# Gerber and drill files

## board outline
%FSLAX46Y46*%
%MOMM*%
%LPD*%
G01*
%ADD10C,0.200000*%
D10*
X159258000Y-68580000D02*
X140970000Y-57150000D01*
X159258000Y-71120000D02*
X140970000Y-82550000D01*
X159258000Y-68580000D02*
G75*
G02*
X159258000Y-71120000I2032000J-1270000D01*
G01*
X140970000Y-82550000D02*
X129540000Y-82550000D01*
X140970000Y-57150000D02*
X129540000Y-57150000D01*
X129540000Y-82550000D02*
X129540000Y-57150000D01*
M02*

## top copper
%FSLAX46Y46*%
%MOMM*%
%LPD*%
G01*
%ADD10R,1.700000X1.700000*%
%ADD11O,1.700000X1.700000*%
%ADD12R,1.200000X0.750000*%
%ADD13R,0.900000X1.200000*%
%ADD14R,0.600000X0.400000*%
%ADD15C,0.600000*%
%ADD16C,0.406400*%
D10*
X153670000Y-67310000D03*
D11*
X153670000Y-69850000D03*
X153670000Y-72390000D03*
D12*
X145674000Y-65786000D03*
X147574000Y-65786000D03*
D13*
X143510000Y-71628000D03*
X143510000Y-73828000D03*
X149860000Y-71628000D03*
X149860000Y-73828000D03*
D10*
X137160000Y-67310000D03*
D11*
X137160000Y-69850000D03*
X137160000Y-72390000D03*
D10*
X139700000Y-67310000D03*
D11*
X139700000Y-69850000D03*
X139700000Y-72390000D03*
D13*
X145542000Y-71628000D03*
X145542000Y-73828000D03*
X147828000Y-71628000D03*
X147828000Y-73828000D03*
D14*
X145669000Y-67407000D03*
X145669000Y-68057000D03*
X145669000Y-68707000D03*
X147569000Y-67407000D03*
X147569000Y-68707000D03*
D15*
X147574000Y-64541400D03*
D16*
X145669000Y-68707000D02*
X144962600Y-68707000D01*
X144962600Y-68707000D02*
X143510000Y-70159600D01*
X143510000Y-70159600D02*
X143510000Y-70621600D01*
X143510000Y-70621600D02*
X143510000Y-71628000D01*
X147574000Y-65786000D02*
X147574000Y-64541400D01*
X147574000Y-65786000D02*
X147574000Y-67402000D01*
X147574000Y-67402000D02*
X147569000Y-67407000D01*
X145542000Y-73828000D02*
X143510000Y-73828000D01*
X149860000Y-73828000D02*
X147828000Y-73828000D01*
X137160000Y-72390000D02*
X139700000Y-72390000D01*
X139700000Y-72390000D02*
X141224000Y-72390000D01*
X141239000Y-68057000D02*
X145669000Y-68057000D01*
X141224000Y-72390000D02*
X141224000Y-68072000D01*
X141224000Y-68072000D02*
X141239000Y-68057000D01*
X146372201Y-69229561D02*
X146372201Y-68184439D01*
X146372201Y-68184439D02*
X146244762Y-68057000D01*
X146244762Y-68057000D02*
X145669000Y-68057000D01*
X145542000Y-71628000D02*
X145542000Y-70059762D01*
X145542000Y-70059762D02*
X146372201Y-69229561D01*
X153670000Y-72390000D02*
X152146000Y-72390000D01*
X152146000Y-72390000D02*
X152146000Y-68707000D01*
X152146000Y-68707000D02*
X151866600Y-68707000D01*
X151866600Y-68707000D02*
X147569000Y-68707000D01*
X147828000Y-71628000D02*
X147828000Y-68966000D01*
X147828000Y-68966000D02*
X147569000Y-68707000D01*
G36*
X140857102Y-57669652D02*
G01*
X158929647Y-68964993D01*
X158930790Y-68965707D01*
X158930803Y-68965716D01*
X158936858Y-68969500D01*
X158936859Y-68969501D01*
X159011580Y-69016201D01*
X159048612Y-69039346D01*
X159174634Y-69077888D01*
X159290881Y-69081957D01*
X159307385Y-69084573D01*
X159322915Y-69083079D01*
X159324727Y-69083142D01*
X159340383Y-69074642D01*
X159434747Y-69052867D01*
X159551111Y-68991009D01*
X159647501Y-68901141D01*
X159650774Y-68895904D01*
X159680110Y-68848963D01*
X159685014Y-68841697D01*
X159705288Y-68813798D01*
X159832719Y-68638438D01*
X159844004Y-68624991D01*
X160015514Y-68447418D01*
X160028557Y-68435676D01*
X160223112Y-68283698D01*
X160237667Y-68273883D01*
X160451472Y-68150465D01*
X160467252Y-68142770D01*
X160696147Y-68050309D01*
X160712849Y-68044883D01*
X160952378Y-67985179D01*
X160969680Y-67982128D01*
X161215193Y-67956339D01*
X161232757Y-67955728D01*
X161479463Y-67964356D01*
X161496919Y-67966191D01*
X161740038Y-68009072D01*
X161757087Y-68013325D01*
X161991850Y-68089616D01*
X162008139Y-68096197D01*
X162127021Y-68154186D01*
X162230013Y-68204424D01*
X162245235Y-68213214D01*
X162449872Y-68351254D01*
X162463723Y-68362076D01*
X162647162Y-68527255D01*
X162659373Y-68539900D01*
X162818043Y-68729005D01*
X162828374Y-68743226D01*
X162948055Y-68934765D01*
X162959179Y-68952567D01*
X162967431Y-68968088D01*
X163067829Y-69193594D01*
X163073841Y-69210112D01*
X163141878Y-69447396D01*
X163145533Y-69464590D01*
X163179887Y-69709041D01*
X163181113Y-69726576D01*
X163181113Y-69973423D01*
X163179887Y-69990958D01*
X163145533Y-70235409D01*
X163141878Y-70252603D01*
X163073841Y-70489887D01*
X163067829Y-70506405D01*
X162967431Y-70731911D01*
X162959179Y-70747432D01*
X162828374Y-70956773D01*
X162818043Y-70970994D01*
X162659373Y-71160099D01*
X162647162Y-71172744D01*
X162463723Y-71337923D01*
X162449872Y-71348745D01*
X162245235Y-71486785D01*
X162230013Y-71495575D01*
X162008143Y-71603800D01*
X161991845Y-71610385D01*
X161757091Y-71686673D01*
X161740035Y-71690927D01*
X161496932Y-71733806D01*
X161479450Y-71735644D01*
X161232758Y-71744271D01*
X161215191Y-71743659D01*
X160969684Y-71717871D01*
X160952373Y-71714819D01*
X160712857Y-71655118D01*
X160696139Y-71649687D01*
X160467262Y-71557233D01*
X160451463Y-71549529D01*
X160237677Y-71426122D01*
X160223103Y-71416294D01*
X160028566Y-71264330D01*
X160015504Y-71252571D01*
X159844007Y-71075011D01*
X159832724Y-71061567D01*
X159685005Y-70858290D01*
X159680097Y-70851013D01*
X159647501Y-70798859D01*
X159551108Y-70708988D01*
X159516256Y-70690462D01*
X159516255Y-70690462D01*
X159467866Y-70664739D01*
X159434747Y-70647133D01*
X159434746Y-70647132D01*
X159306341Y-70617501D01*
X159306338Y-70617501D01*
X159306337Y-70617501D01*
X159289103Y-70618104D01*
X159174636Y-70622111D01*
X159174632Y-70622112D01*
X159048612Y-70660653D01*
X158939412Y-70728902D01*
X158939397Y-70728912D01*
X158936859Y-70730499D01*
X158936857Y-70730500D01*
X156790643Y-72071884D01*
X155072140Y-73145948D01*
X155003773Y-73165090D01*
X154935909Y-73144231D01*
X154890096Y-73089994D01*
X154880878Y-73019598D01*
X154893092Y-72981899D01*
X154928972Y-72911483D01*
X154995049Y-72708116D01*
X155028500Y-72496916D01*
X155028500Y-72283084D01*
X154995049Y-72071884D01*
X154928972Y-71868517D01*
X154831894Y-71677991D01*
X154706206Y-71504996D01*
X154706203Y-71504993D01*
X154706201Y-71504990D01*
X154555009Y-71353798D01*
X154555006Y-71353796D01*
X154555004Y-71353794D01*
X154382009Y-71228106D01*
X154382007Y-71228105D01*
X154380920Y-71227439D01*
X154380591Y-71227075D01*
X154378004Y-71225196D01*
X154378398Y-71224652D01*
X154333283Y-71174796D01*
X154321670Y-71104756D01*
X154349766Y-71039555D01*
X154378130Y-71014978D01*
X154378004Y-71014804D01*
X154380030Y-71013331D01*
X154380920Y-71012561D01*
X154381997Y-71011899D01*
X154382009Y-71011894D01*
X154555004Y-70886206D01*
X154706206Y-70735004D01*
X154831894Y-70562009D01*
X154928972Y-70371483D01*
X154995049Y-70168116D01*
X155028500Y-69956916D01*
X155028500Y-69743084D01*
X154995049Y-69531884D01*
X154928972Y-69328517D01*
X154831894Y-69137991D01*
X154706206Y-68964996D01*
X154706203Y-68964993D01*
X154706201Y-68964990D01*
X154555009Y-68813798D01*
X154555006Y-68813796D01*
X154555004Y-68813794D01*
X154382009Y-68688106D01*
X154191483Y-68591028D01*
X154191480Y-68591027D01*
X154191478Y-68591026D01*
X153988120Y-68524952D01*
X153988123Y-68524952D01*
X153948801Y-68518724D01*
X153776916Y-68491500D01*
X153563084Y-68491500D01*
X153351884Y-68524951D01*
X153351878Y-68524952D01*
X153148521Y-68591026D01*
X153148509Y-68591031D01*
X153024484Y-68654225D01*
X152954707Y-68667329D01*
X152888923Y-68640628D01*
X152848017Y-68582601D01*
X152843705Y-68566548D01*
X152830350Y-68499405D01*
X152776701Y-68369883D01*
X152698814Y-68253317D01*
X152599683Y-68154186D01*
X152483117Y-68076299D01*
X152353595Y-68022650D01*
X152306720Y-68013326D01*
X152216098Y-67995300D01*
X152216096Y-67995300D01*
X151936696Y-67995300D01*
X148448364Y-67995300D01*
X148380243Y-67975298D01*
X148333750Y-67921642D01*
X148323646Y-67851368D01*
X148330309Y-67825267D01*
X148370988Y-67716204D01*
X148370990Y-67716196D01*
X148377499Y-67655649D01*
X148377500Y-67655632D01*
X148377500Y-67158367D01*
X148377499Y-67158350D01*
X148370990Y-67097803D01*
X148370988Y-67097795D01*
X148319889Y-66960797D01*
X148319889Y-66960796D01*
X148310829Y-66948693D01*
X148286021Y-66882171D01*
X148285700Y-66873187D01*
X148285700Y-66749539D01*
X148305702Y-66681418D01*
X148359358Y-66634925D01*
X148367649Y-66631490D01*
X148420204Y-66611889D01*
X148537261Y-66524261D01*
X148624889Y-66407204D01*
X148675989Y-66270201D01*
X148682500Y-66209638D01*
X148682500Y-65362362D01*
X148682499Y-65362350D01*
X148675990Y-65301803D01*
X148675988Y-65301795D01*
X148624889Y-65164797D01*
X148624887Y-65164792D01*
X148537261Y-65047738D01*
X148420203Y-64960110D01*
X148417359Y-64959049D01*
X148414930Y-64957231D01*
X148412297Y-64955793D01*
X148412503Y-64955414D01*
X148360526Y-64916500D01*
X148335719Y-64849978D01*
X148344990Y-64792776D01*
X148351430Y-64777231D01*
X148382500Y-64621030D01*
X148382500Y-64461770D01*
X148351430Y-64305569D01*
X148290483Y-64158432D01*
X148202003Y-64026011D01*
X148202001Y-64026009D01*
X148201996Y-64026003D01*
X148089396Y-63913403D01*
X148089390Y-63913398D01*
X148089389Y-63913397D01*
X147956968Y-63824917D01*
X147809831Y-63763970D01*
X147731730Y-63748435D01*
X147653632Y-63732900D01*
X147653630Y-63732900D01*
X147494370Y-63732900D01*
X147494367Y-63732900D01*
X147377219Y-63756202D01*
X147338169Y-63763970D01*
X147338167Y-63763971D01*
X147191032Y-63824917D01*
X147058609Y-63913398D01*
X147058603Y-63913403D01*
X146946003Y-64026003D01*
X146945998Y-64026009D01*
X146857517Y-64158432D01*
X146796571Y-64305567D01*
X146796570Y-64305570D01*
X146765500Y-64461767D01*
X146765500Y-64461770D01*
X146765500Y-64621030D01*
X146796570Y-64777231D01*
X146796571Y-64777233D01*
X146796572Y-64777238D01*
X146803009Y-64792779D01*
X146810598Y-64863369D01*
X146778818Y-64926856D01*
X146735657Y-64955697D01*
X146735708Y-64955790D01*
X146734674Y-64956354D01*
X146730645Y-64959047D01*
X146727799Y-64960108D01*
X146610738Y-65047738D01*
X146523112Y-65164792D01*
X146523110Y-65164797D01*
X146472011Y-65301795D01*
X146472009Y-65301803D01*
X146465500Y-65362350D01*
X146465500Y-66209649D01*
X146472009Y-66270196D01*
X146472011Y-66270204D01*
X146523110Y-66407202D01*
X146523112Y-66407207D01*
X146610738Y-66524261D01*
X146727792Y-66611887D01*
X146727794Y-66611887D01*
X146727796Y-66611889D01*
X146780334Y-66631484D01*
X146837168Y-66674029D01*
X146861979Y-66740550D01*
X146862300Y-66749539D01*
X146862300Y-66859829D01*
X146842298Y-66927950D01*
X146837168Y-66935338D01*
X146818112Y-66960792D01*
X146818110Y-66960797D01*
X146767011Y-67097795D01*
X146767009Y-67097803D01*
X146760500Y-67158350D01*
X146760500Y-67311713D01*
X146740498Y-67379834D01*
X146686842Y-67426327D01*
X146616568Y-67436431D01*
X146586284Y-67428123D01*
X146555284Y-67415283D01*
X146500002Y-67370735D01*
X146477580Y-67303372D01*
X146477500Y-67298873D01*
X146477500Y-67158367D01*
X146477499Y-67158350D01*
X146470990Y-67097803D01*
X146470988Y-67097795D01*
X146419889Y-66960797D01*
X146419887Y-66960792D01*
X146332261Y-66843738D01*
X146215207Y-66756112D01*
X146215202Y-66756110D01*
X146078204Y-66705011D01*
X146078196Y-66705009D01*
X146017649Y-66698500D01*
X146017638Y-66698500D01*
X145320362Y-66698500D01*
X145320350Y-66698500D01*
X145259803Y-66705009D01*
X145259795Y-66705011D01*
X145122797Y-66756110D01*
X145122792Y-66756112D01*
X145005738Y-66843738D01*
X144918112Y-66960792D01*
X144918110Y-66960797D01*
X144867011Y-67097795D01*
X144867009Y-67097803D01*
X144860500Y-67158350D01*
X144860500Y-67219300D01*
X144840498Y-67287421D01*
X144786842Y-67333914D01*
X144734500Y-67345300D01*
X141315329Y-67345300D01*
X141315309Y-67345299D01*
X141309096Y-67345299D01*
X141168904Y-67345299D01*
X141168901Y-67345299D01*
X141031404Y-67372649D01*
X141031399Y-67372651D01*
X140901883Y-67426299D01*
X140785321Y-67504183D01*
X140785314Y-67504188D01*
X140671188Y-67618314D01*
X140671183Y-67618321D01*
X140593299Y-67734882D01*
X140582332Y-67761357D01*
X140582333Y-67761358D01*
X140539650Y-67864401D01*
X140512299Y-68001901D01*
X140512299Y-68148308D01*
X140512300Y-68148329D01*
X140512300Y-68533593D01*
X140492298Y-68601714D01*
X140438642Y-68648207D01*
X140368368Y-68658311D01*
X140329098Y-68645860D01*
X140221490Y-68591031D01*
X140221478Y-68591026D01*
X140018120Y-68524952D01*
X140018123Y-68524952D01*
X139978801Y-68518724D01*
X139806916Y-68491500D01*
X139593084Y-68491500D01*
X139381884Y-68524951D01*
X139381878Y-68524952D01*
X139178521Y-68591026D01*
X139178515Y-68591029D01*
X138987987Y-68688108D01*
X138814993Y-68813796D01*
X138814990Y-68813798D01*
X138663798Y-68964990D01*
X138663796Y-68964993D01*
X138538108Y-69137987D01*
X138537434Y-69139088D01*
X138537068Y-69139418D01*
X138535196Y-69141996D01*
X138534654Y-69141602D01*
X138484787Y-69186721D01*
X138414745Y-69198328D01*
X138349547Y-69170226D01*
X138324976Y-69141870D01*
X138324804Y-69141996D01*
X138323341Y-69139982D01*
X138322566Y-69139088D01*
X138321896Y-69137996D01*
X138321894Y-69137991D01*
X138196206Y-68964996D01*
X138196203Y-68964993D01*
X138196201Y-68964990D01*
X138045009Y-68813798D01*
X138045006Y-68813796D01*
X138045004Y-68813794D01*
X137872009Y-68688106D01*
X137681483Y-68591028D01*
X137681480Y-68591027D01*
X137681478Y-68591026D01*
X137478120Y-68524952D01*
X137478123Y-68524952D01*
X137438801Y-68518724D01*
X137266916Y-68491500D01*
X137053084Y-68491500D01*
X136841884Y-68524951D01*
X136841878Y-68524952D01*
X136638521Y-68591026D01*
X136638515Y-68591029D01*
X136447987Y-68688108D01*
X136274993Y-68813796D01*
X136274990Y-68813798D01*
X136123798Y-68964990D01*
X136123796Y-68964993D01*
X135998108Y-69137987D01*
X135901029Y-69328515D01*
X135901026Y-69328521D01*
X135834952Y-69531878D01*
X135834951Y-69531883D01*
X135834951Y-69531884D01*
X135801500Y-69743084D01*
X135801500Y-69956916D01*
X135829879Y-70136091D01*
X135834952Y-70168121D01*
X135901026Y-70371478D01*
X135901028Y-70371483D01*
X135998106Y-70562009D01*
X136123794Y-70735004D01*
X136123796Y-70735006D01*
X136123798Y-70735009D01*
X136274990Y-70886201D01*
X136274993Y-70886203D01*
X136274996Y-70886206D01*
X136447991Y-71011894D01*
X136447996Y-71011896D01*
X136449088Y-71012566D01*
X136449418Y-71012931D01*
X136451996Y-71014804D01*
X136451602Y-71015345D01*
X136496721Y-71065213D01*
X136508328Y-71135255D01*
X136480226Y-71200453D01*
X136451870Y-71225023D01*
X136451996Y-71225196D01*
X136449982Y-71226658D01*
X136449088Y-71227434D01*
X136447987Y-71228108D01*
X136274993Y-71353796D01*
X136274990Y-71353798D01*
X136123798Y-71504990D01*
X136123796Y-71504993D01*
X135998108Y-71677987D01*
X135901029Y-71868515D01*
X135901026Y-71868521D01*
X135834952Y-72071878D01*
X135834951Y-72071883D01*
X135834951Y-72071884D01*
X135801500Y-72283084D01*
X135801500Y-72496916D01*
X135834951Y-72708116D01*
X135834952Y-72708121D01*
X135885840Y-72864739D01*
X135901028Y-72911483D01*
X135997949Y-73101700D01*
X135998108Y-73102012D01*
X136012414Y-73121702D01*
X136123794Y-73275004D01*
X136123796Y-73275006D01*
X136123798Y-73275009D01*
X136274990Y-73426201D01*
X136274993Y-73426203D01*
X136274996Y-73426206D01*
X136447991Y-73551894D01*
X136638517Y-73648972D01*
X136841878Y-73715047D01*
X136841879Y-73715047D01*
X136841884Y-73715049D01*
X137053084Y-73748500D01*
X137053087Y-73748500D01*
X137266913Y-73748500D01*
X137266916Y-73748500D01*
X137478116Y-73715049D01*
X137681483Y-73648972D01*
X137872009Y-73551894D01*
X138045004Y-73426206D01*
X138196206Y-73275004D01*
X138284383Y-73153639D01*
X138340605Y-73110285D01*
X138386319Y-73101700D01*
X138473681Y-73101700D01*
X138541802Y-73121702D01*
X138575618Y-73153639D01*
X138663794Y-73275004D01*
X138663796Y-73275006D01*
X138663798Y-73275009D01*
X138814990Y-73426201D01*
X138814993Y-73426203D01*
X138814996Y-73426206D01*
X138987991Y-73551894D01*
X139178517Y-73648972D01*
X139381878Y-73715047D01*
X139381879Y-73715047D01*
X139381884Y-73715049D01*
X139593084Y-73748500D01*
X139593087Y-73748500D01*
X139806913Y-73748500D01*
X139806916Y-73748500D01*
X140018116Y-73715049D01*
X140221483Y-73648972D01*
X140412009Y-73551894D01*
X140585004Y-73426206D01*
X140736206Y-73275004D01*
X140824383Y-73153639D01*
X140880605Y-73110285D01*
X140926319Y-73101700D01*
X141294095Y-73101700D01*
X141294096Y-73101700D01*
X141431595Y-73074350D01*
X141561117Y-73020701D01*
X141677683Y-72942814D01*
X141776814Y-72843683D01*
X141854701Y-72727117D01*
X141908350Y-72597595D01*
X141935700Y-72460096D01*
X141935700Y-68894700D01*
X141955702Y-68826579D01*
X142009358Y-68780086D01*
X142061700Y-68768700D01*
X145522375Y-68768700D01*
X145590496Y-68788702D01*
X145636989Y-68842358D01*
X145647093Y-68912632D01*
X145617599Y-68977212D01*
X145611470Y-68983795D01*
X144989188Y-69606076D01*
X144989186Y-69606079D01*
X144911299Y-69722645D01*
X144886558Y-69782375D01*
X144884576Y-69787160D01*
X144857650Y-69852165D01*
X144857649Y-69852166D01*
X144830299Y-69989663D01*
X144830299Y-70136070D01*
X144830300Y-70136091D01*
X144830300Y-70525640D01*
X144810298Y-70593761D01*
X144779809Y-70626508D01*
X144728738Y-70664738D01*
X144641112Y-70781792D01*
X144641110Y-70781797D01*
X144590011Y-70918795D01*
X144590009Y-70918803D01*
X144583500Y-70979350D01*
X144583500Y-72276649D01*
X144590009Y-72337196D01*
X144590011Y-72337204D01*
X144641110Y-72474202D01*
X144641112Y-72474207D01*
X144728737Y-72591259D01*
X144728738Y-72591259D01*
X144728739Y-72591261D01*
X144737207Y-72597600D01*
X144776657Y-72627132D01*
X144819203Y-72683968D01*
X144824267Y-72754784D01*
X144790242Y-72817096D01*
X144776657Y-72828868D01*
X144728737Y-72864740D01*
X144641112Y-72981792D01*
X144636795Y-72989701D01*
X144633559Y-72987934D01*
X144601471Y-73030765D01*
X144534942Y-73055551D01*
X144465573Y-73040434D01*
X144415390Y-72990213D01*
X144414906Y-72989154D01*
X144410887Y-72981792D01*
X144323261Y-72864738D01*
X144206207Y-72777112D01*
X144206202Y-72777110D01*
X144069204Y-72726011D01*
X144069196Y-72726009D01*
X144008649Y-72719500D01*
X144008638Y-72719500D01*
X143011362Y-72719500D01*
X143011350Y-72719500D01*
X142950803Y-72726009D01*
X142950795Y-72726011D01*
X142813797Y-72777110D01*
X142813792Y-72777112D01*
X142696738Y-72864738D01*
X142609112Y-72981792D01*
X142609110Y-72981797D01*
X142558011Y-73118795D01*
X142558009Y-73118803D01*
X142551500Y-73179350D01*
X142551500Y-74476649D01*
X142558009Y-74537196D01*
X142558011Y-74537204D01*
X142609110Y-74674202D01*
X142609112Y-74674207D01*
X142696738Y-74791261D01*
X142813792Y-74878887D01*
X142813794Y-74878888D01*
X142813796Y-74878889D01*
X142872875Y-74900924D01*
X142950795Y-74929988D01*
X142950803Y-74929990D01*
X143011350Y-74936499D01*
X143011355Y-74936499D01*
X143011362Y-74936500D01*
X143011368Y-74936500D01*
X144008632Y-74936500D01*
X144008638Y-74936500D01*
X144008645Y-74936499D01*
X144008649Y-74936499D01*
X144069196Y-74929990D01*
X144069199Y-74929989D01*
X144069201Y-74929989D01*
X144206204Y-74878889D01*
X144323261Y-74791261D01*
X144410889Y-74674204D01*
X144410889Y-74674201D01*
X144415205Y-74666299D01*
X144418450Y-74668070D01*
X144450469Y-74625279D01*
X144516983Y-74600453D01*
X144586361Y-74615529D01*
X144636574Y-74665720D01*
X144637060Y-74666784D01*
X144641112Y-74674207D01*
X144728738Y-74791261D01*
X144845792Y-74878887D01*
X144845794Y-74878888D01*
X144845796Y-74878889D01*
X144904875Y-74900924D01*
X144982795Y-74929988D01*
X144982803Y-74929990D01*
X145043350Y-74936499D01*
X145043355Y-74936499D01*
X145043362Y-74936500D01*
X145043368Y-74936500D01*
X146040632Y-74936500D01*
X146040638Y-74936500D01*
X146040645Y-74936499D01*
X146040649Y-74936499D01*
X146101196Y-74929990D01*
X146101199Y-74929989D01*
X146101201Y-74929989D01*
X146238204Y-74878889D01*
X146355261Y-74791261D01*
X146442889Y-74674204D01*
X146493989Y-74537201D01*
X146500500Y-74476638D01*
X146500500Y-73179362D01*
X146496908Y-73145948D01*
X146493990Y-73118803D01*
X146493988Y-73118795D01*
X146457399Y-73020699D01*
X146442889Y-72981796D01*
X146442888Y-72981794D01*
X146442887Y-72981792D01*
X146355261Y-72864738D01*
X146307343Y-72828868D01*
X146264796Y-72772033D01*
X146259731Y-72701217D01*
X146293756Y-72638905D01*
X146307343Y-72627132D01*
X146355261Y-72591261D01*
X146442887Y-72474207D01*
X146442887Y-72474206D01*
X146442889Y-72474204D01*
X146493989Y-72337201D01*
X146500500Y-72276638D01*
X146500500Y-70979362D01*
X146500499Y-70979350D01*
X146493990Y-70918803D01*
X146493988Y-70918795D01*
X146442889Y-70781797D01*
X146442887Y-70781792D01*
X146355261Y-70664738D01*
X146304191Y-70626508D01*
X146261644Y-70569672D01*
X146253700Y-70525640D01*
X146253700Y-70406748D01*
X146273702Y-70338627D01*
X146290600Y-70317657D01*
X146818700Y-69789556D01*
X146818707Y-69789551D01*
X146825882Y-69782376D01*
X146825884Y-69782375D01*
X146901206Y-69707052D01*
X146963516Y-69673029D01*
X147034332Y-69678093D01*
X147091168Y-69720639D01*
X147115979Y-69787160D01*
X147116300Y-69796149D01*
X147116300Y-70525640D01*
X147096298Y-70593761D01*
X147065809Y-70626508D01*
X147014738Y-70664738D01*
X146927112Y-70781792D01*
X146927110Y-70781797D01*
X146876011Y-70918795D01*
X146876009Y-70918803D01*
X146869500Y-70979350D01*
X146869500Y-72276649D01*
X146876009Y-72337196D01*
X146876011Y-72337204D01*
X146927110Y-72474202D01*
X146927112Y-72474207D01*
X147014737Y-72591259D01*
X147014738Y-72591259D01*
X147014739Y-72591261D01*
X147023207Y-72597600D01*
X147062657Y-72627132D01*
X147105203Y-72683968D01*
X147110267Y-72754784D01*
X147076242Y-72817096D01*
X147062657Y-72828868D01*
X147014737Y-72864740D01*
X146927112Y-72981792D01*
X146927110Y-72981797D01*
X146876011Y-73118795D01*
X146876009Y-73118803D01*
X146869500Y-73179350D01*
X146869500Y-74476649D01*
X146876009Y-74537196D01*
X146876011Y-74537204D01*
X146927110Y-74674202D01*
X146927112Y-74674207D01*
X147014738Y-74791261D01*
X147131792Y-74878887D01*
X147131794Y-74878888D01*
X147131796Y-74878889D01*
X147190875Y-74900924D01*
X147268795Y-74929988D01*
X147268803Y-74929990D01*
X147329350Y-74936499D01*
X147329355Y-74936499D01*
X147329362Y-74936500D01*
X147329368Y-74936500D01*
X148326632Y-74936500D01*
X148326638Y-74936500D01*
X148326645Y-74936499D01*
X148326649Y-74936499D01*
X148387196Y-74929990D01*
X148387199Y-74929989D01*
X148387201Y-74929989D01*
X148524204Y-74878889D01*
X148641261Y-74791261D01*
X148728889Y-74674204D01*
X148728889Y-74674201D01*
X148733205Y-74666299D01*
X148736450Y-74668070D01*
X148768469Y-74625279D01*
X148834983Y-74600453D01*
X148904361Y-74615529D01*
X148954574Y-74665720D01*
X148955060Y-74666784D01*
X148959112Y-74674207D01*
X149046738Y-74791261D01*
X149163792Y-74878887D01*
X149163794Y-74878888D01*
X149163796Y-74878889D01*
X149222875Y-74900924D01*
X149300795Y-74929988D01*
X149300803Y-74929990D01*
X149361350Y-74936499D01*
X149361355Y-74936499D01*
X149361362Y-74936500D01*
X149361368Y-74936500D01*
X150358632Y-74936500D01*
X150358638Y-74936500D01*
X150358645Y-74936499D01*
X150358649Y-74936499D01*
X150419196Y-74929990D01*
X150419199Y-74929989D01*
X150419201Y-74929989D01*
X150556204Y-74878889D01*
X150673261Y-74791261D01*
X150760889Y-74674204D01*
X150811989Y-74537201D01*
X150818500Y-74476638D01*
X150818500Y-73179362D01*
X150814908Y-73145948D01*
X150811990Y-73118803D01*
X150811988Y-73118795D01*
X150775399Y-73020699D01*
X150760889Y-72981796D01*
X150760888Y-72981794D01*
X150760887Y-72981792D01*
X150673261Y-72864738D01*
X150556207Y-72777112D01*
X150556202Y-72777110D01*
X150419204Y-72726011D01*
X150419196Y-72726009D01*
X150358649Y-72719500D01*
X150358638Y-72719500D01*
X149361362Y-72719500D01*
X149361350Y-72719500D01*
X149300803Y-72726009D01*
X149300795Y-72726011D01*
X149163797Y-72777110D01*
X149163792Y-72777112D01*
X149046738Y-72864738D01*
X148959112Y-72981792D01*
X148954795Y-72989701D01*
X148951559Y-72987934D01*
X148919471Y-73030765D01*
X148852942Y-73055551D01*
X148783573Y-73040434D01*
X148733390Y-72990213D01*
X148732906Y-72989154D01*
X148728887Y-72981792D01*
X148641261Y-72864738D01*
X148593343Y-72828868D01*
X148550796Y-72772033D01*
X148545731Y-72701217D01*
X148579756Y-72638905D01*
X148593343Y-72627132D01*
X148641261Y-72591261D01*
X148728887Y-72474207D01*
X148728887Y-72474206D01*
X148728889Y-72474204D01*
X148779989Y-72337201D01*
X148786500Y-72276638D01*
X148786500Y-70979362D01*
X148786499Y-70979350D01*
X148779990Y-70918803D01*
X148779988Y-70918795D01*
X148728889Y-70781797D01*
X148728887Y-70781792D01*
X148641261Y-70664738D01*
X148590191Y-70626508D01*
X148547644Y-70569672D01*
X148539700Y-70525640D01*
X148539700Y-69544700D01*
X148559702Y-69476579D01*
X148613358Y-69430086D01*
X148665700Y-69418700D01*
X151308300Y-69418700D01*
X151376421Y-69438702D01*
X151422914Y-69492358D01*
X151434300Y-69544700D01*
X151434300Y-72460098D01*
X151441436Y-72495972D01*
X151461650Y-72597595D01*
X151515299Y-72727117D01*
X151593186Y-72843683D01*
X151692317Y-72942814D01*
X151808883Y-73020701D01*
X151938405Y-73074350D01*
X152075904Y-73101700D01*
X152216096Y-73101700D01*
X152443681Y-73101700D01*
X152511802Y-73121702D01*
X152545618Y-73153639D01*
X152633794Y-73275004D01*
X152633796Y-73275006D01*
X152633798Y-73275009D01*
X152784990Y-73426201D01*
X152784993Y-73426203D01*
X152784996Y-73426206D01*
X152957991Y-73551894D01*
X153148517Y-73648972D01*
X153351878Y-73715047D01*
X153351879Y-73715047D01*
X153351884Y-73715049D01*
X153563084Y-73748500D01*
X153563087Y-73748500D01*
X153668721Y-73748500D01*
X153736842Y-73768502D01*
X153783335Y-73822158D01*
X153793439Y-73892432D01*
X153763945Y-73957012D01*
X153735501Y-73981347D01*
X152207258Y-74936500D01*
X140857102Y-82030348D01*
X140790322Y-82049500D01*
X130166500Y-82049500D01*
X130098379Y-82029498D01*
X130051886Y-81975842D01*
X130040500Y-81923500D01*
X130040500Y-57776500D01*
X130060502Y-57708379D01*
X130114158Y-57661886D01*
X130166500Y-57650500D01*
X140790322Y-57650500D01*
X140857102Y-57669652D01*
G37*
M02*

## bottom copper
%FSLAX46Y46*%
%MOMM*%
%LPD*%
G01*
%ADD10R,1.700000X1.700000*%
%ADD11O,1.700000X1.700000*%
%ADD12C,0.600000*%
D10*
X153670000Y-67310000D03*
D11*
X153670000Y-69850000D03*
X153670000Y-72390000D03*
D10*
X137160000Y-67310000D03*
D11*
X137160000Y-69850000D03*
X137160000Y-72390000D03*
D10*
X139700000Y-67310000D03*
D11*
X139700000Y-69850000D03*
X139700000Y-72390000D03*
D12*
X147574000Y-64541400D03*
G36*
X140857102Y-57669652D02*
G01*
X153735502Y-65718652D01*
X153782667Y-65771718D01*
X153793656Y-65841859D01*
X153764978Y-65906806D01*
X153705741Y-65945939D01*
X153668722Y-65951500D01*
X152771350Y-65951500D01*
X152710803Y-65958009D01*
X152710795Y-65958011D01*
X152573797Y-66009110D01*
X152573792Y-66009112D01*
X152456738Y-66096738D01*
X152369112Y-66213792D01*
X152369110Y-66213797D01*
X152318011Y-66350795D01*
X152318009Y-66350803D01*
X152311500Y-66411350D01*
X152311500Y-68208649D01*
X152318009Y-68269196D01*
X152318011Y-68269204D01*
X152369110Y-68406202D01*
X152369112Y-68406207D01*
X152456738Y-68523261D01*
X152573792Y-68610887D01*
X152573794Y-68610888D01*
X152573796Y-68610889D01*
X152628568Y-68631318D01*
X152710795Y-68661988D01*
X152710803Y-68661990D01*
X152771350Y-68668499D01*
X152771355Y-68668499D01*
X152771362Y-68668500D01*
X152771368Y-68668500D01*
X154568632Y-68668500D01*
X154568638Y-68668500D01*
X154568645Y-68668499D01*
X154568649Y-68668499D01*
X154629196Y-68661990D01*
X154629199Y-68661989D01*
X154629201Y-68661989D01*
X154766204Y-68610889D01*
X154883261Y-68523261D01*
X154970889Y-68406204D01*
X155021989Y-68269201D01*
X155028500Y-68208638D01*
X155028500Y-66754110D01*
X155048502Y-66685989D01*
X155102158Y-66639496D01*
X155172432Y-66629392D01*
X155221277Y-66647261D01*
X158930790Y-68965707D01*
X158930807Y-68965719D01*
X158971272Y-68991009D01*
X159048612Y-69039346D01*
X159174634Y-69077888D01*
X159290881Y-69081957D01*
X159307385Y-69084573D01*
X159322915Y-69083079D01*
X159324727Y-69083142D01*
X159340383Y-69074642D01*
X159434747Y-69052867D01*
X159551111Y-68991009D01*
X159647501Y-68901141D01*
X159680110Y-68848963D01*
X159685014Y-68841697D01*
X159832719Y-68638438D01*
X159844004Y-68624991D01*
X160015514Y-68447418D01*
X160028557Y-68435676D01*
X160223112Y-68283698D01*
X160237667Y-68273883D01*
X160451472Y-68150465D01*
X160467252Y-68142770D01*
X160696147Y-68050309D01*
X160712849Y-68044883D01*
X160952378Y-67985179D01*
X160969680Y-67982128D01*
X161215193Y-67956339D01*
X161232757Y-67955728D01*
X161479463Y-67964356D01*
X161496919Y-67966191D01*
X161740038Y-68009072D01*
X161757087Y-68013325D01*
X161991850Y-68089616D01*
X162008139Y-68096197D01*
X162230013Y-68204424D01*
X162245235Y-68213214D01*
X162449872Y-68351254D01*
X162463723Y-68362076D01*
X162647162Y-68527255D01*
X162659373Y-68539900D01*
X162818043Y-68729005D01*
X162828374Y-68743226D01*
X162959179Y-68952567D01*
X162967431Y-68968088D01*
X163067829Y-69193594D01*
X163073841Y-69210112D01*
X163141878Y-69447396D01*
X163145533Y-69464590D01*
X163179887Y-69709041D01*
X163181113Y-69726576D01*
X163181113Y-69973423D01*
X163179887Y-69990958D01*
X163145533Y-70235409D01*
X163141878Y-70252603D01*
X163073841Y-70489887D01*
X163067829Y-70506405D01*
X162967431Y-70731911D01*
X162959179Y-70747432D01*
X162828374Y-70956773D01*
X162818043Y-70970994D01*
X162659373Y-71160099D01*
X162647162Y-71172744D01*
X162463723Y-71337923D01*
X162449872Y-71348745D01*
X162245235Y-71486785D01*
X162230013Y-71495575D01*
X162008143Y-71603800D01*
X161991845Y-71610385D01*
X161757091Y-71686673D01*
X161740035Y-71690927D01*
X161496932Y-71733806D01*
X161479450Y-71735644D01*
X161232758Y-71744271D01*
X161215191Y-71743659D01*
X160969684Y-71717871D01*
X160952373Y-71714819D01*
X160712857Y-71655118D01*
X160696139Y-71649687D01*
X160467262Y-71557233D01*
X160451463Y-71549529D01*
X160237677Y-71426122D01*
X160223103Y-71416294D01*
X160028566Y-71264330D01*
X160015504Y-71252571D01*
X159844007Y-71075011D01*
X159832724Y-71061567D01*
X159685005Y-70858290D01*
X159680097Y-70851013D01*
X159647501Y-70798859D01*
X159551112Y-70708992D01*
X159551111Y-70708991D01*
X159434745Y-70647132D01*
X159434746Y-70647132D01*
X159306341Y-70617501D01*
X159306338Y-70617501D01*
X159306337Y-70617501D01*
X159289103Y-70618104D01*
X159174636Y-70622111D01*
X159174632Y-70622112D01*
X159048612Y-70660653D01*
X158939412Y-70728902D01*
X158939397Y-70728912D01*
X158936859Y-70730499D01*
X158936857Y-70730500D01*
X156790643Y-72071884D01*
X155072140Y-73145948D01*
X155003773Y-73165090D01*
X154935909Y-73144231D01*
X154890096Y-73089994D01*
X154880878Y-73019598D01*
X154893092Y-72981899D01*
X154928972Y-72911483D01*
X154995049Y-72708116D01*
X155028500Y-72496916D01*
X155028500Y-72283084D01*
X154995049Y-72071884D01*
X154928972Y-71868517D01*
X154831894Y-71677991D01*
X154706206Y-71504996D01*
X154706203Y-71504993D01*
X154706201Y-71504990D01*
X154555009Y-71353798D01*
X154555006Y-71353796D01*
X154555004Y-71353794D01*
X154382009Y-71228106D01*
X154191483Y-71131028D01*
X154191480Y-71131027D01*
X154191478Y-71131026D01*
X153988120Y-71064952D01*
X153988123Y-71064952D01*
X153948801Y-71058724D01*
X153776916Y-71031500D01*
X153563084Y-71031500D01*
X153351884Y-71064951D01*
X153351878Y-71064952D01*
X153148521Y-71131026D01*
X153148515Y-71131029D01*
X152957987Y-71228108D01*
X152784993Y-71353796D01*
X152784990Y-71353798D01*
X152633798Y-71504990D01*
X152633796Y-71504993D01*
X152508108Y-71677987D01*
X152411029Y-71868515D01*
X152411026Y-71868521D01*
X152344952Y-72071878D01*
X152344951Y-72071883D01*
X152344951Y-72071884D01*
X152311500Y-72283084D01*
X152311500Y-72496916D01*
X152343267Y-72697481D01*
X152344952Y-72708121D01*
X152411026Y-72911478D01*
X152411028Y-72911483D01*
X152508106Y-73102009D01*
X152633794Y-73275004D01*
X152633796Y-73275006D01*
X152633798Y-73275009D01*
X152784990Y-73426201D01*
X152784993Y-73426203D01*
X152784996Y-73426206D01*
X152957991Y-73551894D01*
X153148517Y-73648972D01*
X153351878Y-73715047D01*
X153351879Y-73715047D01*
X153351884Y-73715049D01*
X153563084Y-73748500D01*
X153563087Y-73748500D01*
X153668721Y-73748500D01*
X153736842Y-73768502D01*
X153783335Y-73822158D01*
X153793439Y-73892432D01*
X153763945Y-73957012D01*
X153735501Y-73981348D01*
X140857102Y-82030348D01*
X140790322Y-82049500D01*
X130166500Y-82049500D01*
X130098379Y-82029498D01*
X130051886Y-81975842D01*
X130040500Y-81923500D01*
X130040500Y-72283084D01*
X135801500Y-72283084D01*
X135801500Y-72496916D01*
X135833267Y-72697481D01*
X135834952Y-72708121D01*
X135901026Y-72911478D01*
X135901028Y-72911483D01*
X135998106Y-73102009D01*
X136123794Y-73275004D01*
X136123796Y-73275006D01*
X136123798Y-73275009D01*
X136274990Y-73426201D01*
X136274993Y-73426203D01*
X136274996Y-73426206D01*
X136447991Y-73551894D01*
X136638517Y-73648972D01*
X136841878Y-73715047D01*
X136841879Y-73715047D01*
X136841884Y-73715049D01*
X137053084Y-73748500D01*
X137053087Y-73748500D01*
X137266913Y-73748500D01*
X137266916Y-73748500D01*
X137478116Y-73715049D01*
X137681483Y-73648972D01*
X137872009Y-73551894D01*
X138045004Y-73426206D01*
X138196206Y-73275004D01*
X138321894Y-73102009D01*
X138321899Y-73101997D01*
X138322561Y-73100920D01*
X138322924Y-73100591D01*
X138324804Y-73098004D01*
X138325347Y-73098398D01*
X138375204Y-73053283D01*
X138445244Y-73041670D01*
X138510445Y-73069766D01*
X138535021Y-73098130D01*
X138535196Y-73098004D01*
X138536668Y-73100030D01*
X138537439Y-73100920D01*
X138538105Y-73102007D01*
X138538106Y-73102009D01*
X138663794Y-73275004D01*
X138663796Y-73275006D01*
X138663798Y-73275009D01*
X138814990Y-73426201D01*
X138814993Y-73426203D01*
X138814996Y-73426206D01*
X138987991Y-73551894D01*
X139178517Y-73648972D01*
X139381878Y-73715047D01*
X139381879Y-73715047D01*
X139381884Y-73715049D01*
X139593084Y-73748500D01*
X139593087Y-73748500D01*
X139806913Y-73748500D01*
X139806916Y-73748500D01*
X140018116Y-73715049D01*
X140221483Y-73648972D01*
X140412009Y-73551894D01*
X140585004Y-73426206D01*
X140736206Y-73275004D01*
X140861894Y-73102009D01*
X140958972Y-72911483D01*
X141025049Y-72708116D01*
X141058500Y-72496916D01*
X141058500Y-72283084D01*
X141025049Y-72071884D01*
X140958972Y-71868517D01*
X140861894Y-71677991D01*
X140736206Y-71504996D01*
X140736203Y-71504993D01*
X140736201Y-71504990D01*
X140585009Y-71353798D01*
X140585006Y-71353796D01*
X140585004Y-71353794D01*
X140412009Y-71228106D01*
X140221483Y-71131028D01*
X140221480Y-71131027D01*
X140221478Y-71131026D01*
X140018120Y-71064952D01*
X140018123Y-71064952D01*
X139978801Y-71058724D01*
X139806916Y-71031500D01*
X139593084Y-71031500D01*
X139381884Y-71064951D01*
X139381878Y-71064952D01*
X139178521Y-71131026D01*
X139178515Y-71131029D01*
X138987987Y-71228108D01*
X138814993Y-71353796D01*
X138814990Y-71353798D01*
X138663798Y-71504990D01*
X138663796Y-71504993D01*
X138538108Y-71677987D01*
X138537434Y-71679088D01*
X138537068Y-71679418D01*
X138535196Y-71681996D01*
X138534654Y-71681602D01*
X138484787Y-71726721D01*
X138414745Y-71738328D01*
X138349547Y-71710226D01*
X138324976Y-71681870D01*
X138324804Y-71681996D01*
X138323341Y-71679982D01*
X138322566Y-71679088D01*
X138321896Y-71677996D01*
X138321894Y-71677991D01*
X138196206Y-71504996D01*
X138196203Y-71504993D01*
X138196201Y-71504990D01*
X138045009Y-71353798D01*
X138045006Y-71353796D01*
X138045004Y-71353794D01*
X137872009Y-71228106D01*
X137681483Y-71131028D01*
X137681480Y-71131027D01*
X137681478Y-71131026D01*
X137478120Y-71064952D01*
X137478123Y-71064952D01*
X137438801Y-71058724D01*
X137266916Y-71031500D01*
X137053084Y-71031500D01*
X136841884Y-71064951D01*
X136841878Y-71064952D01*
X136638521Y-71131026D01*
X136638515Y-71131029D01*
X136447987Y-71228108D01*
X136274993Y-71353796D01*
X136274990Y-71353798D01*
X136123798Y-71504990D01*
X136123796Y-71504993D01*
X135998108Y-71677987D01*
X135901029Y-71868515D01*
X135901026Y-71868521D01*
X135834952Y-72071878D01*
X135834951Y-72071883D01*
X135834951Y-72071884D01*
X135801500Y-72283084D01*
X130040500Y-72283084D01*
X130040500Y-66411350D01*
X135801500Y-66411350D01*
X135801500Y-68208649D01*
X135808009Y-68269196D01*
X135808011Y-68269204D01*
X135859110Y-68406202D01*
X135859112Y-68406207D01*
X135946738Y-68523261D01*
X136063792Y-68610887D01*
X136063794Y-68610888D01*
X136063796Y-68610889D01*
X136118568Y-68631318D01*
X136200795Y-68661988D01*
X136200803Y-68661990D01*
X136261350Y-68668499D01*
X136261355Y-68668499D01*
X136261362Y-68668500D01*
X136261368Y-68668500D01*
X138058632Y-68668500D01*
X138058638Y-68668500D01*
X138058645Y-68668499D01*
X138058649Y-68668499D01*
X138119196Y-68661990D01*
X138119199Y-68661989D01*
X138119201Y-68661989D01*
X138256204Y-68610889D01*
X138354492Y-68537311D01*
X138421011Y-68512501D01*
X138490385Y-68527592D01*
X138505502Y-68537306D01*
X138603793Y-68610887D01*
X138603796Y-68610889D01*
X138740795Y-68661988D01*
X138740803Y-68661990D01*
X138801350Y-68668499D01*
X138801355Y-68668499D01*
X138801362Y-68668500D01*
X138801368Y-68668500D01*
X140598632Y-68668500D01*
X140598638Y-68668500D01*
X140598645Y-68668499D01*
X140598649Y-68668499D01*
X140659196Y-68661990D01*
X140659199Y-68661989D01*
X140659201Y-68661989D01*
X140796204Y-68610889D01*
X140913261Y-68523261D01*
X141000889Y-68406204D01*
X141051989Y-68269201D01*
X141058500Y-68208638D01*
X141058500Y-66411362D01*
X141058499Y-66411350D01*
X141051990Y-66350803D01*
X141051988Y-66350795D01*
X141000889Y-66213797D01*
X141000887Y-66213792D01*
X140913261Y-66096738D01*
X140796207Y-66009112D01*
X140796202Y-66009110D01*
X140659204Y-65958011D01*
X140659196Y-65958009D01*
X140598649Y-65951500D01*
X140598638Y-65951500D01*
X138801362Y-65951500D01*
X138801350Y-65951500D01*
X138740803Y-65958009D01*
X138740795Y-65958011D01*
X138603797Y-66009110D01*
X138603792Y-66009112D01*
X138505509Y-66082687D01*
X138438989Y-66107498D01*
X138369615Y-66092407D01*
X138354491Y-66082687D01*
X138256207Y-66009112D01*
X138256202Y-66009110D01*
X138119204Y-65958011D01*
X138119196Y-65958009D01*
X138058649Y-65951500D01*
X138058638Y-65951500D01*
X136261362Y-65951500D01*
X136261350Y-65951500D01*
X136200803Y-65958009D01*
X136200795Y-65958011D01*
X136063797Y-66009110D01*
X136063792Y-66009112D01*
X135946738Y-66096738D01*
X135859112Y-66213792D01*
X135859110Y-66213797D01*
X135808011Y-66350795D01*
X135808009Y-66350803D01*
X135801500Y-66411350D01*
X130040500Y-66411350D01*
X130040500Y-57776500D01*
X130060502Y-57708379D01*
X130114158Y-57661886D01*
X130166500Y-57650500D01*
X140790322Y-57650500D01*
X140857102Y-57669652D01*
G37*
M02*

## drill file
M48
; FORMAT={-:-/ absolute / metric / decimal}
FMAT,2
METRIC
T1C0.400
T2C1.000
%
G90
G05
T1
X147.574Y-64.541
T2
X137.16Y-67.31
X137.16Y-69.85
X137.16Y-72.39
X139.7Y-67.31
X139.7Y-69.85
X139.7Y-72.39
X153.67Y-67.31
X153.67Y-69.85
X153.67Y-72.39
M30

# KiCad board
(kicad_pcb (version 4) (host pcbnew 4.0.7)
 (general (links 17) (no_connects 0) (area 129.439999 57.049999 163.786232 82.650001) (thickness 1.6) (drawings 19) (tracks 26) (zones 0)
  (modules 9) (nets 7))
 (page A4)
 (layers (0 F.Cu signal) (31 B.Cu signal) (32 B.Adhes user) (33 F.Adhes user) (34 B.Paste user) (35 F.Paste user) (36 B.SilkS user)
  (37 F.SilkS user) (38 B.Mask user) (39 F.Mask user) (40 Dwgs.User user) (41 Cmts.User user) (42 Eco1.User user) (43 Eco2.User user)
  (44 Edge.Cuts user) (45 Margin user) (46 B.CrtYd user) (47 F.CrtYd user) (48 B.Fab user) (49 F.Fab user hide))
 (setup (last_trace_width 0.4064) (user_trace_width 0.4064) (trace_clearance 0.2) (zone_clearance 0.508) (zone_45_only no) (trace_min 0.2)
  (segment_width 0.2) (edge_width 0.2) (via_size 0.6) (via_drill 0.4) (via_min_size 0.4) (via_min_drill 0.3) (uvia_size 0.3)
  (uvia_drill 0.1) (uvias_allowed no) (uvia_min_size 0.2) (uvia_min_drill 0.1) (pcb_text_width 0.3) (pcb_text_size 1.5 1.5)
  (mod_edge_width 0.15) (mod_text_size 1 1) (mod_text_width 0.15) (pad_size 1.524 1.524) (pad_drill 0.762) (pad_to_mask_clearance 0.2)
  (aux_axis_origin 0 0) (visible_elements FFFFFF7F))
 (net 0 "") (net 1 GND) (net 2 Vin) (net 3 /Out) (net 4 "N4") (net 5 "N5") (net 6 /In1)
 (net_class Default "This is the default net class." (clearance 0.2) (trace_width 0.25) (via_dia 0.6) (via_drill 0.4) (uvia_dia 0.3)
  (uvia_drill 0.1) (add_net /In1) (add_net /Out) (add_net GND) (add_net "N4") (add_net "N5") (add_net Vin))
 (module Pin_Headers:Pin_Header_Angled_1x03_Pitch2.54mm (layer F.Cu) (at 153.67 67.31)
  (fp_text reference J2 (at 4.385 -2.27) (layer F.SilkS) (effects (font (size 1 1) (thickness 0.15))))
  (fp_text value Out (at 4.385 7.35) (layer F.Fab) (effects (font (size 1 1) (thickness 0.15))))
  (pad 1 thru_hole rect (at 0 0) (size 1.7 1.7) (drill 1) (layers *.Cu *.Mask) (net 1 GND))
  (pad 2 thru_hole oval (at 0 2.54) (size 1.7 1.7) (drill 1) (layers *.Cu *.Mask) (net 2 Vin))
  (pad 3 thru_hole oval (at 0 5.08) (size 1.7 1.7) (drill 1) (layers *.Cu *.Mask) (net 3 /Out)))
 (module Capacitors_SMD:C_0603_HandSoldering (layer F.Cu) (at 146.624 65.786)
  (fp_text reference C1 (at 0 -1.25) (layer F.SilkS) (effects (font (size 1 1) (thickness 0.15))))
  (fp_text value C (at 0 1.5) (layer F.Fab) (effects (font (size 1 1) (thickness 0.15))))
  (pad 1 smd rect (at -0.95 0) (size 1.2 0.75) (layers F.Cu F.Paste F.Mask) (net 1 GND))
  (pad 2 smd rect (at 0.95 0) (size 1.2 0.75) (layers F.Cu F.Paste F.Mask) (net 2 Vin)))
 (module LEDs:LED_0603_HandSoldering (layer F.Cu) (at 143.51 72.728 270)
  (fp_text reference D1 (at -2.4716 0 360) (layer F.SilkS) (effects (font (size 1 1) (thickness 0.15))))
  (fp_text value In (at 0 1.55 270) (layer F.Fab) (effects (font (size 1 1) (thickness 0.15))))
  (pad 1 smd rect (at -1.1 0 270) (size 1.2 0.9) (layers F.Cu F.Paste F.Mask) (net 1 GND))
  (pad 2 smd rect (at 1.1 0 270) (size 1.2 0.9) (layers F.Cu F.Paste F.Mask) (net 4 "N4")))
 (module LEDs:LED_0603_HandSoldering (layer F.Cu) (at 149.86 72.728 270)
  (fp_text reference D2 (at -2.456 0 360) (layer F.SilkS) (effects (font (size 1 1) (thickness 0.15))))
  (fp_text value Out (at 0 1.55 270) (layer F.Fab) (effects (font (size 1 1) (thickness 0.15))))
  (pad 1 smd rect (at -1.1 0 270) (size 1.2 0.9) (layers F.Cu F.Paste F.Mask) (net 1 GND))
  (pad 2 smd rect (at 1.1 0 270) (size 1.2 0.9) (layers F.Cu F.Paste F.Mask) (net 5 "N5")))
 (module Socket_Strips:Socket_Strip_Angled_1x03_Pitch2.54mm (layer F.Cu) (at 137.16 67.31)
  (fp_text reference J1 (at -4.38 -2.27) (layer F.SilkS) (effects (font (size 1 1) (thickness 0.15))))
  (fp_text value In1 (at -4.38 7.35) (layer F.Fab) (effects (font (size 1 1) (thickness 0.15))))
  (pad 1 thru_hole rect (at 0 0) (size 1.7 1.7) (drill 1) (layers *.Cu *.Mask) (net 1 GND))
  (pad 2 thru_hole oval (at 0 2.54) (size 1.7 1.7) (drill 1) (layers *.Cu *.Mask) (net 2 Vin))
  (pad 3 thru_hole oval (at 0 5.08) (size 1.7 1.7) (drill 1) (layers *.Cu *.Mask) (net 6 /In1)))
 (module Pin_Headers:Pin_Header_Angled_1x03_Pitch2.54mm (layer B.Cu) (at 139.7 67.31 180)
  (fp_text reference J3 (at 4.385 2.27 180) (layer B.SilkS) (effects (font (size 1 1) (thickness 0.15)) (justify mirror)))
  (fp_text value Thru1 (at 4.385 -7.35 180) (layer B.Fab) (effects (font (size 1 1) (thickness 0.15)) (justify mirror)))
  (pad 1 thru_hole rect (at 0 0 180) (size 1.7 1.7) (drill 1) (layers *.Cu *.Mask) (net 1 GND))
  (pad 2 thru_hole oval (at 0 -2.54 180) (size 1.7 1.7) (drill 1) (layers *.Cu *.Mask) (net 2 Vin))
  (pad 3 thru_hole oval (at 0 -5.08 180) (size 1.7 1.7) (drill 1) (layers *.Cu *.Mask) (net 6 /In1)))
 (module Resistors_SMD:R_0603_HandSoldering (layer F.Cu) (at 145.542 72.728 270)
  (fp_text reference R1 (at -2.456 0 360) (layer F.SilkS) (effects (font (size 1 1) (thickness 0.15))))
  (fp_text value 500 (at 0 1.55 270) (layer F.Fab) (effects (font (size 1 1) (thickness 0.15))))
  (pad 1 smd rect (at -1.1 0 270) (size 1.2 0.9) (layers F.Cu F.Paste F.Mask) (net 6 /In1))
  (pad 2 smd rect (at 1.1 0 270) (size 1.2 0.9) (layers F.Cu F.Paste F.Mask) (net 4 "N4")))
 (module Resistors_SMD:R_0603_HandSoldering (layer F.Cu) (at 147.828 72.728 270)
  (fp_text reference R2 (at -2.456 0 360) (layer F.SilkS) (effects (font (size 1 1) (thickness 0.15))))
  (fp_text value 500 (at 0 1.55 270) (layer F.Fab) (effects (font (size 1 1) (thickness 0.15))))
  (pad 1 smd rect (at -1.1 0 270) (size 1.2 0.9) (layers F.Cu F.Paste F.Mask) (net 3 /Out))
  (pad 2 smd rect (at 1.1 0 270) (size 1.2 0.9) (layers F.Cu F.Paste F.Mask) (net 5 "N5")))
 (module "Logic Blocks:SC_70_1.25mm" (layer F.Cu) (at 146.05 67.1276 270)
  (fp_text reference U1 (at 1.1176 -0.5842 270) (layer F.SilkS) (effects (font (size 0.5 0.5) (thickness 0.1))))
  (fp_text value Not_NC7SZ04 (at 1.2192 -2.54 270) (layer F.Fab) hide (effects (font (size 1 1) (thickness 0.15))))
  (pad 1 smd rect (at 0.2794 0.381 270) (size 0.4 0.6) (layers F.Cu F.Paste F.Mask))
  (pad 2 smd rect (at 0.9294 0.381 270) (size 0.4 0.6) (layers F.Cu F.Paste F.Mask) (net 6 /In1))
  (pad 3 smd rect (at 1.5794 0.381 270) (size 0.4 0.6) (layers F.Cu F.Paste F.Mask) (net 1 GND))
  (pad 5 smd rect (at 0.2794 -1.519 270) (size 0.4 0.6) (layers F.Cu F.Paste F.Mask) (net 2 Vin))
  (pad 4 smd rect (at 1.5794 -1.519 270) (size 0.4 0.6) (layers F.Cu F.Paste F.Mask) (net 3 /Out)))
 (gr_line (start 159.258 68.58) (end 140.97 57.15) (layer Edge.Cuts) (width 0.2))
 (gr_line (start 159.258 71.12) (end 140.97 82.55) (layer Edge.Cuts) (width 0.2))
 (gr_arc (start 161.29 69.85) (end 159.258 68.58) (angle 295.9892336) (layer Edge.Cuts) (width 0.2))
 (gr_line (start 140.97 82.55) (end 129.54 82.55) (layer Edge.Cuts) (width 0.2))
 (gr_line (start 140.97 57.15) (end 129.54 57.15) (layer Edge.Cuts) (width 0.2))
 (gr_line (start 129.54 82.55) (end 129.54 57.15) (layer Edge.Cuts) (width 0.2))
 (segment (start 145.669 68.707) (end 144.9626 68.707) (width 0.4064) (layer F.Cu) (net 1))
 (segment (start 144.9626 68.707) (end 143.51 70.1596) (width 0.4064) (layer F.Cu) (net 1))
 (segment (start 143.51 70.1596) (end 143.51 70.6216) (width 0.4064) (layer F.Cu) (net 1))
 (segment (start 143.51 70.6216) (end 143.51 71.628) (width 0.4064) (layer F.Cu) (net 1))
 (segment (start 147.574 65.786) (end 147.574 64.5414) (width 0.4064) (layer F.Cu) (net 2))
 (via (at 147.574 64.5414) (size 0.6) (drill 0.4) (layers F.Cu B.Cu) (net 2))
 (segment (start 147.574 65.786) (end 147.574 67.402) (width 0.4064) (layer F.Cu) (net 2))
 (segment (start 147.574 67.402) (end 147.569 67.407) (width 0.4064) (layer F.Cu) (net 2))
 (segment (start 145.542 73.828) (end 143.51 73.828) (width 0.4064) (layer F.Cu) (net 4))
 (segment (start 149.86 73.828) (end 147.828 73.828) (width 0.4064) (layer F.Cu) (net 5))
 (segment (start 137.16 72.39) (end 139.7 72.39) (width 0.4064) (layer F.Cu) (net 6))
 (segment (start 139.7 72.39) (end 141.224 72.39) (width 0.4064) (layer F.Cu) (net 6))
 (segment (start 141.239 68.057) (end 145.669 68.057) (width 0.4064) (layer F.Cu) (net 6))
 (segment (start 141.224 72.39) (end 141.224 68.072) (width 0.4064) (layer F.Cu) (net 6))
 (segment (start 141.224 68.072) (end 141.239 68.057) (width 0.4064) (layer F.Cu) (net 6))
 (segment (start 146.372201 69.229561) (end 146.372201 68.184439) (width 0.4064) (layer F.Cu) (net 6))
 (segment (start 146.372201 68.184439) (end 146.244762 68.057) (width 0.4064) (layer F.Cu) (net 6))
 (segment (start 146.244762 68.057) (end 145.669 68.057) (width 0.4064) (layer F.Cu) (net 6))
 (segment (start 145.542 71.628) (end 145.542 70.059762) (width 0.4064) (layer F.Cu) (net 6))
 (segment (start 145.542 70.059762) (end 146.372201 69.229561) (width 0.4064) (layer F.Cu) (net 6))
 (segment (start 153.67 72.39) (end 152.146 72.39) (width 0.4064) (layer F.Cu) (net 3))
 (segment (start 152.146 72.39) (end 152.146 68.707) (width 0.4064) (layer F.Cu) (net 3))
 (segment (start 152.146 68.707) (end 151.8666 68.707) (width 0.4064) (layer F.Cu) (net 3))
 (segment (start 151.8666 68.707) (end 147.569 68.707) (width 0.4064) (layer F.Cu) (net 3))
 (segment (start 147.828 71.628) (end 147.828 68.966) (width 0.4064) (layer F.Cu) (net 3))
 (segment (start 147.828 68.966) (end 147.569 68.707) (width 0.4064) (layer F.Cu) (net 3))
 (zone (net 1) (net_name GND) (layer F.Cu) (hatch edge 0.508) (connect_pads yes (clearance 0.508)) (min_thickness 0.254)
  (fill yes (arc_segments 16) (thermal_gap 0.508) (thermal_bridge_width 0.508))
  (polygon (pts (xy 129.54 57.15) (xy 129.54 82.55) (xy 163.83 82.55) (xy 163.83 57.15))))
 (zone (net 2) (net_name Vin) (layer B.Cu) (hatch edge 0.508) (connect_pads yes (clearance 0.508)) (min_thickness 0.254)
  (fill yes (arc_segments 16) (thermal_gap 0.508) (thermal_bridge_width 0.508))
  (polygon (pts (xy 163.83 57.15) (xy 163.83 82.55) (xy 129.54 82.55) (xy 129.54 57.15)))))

